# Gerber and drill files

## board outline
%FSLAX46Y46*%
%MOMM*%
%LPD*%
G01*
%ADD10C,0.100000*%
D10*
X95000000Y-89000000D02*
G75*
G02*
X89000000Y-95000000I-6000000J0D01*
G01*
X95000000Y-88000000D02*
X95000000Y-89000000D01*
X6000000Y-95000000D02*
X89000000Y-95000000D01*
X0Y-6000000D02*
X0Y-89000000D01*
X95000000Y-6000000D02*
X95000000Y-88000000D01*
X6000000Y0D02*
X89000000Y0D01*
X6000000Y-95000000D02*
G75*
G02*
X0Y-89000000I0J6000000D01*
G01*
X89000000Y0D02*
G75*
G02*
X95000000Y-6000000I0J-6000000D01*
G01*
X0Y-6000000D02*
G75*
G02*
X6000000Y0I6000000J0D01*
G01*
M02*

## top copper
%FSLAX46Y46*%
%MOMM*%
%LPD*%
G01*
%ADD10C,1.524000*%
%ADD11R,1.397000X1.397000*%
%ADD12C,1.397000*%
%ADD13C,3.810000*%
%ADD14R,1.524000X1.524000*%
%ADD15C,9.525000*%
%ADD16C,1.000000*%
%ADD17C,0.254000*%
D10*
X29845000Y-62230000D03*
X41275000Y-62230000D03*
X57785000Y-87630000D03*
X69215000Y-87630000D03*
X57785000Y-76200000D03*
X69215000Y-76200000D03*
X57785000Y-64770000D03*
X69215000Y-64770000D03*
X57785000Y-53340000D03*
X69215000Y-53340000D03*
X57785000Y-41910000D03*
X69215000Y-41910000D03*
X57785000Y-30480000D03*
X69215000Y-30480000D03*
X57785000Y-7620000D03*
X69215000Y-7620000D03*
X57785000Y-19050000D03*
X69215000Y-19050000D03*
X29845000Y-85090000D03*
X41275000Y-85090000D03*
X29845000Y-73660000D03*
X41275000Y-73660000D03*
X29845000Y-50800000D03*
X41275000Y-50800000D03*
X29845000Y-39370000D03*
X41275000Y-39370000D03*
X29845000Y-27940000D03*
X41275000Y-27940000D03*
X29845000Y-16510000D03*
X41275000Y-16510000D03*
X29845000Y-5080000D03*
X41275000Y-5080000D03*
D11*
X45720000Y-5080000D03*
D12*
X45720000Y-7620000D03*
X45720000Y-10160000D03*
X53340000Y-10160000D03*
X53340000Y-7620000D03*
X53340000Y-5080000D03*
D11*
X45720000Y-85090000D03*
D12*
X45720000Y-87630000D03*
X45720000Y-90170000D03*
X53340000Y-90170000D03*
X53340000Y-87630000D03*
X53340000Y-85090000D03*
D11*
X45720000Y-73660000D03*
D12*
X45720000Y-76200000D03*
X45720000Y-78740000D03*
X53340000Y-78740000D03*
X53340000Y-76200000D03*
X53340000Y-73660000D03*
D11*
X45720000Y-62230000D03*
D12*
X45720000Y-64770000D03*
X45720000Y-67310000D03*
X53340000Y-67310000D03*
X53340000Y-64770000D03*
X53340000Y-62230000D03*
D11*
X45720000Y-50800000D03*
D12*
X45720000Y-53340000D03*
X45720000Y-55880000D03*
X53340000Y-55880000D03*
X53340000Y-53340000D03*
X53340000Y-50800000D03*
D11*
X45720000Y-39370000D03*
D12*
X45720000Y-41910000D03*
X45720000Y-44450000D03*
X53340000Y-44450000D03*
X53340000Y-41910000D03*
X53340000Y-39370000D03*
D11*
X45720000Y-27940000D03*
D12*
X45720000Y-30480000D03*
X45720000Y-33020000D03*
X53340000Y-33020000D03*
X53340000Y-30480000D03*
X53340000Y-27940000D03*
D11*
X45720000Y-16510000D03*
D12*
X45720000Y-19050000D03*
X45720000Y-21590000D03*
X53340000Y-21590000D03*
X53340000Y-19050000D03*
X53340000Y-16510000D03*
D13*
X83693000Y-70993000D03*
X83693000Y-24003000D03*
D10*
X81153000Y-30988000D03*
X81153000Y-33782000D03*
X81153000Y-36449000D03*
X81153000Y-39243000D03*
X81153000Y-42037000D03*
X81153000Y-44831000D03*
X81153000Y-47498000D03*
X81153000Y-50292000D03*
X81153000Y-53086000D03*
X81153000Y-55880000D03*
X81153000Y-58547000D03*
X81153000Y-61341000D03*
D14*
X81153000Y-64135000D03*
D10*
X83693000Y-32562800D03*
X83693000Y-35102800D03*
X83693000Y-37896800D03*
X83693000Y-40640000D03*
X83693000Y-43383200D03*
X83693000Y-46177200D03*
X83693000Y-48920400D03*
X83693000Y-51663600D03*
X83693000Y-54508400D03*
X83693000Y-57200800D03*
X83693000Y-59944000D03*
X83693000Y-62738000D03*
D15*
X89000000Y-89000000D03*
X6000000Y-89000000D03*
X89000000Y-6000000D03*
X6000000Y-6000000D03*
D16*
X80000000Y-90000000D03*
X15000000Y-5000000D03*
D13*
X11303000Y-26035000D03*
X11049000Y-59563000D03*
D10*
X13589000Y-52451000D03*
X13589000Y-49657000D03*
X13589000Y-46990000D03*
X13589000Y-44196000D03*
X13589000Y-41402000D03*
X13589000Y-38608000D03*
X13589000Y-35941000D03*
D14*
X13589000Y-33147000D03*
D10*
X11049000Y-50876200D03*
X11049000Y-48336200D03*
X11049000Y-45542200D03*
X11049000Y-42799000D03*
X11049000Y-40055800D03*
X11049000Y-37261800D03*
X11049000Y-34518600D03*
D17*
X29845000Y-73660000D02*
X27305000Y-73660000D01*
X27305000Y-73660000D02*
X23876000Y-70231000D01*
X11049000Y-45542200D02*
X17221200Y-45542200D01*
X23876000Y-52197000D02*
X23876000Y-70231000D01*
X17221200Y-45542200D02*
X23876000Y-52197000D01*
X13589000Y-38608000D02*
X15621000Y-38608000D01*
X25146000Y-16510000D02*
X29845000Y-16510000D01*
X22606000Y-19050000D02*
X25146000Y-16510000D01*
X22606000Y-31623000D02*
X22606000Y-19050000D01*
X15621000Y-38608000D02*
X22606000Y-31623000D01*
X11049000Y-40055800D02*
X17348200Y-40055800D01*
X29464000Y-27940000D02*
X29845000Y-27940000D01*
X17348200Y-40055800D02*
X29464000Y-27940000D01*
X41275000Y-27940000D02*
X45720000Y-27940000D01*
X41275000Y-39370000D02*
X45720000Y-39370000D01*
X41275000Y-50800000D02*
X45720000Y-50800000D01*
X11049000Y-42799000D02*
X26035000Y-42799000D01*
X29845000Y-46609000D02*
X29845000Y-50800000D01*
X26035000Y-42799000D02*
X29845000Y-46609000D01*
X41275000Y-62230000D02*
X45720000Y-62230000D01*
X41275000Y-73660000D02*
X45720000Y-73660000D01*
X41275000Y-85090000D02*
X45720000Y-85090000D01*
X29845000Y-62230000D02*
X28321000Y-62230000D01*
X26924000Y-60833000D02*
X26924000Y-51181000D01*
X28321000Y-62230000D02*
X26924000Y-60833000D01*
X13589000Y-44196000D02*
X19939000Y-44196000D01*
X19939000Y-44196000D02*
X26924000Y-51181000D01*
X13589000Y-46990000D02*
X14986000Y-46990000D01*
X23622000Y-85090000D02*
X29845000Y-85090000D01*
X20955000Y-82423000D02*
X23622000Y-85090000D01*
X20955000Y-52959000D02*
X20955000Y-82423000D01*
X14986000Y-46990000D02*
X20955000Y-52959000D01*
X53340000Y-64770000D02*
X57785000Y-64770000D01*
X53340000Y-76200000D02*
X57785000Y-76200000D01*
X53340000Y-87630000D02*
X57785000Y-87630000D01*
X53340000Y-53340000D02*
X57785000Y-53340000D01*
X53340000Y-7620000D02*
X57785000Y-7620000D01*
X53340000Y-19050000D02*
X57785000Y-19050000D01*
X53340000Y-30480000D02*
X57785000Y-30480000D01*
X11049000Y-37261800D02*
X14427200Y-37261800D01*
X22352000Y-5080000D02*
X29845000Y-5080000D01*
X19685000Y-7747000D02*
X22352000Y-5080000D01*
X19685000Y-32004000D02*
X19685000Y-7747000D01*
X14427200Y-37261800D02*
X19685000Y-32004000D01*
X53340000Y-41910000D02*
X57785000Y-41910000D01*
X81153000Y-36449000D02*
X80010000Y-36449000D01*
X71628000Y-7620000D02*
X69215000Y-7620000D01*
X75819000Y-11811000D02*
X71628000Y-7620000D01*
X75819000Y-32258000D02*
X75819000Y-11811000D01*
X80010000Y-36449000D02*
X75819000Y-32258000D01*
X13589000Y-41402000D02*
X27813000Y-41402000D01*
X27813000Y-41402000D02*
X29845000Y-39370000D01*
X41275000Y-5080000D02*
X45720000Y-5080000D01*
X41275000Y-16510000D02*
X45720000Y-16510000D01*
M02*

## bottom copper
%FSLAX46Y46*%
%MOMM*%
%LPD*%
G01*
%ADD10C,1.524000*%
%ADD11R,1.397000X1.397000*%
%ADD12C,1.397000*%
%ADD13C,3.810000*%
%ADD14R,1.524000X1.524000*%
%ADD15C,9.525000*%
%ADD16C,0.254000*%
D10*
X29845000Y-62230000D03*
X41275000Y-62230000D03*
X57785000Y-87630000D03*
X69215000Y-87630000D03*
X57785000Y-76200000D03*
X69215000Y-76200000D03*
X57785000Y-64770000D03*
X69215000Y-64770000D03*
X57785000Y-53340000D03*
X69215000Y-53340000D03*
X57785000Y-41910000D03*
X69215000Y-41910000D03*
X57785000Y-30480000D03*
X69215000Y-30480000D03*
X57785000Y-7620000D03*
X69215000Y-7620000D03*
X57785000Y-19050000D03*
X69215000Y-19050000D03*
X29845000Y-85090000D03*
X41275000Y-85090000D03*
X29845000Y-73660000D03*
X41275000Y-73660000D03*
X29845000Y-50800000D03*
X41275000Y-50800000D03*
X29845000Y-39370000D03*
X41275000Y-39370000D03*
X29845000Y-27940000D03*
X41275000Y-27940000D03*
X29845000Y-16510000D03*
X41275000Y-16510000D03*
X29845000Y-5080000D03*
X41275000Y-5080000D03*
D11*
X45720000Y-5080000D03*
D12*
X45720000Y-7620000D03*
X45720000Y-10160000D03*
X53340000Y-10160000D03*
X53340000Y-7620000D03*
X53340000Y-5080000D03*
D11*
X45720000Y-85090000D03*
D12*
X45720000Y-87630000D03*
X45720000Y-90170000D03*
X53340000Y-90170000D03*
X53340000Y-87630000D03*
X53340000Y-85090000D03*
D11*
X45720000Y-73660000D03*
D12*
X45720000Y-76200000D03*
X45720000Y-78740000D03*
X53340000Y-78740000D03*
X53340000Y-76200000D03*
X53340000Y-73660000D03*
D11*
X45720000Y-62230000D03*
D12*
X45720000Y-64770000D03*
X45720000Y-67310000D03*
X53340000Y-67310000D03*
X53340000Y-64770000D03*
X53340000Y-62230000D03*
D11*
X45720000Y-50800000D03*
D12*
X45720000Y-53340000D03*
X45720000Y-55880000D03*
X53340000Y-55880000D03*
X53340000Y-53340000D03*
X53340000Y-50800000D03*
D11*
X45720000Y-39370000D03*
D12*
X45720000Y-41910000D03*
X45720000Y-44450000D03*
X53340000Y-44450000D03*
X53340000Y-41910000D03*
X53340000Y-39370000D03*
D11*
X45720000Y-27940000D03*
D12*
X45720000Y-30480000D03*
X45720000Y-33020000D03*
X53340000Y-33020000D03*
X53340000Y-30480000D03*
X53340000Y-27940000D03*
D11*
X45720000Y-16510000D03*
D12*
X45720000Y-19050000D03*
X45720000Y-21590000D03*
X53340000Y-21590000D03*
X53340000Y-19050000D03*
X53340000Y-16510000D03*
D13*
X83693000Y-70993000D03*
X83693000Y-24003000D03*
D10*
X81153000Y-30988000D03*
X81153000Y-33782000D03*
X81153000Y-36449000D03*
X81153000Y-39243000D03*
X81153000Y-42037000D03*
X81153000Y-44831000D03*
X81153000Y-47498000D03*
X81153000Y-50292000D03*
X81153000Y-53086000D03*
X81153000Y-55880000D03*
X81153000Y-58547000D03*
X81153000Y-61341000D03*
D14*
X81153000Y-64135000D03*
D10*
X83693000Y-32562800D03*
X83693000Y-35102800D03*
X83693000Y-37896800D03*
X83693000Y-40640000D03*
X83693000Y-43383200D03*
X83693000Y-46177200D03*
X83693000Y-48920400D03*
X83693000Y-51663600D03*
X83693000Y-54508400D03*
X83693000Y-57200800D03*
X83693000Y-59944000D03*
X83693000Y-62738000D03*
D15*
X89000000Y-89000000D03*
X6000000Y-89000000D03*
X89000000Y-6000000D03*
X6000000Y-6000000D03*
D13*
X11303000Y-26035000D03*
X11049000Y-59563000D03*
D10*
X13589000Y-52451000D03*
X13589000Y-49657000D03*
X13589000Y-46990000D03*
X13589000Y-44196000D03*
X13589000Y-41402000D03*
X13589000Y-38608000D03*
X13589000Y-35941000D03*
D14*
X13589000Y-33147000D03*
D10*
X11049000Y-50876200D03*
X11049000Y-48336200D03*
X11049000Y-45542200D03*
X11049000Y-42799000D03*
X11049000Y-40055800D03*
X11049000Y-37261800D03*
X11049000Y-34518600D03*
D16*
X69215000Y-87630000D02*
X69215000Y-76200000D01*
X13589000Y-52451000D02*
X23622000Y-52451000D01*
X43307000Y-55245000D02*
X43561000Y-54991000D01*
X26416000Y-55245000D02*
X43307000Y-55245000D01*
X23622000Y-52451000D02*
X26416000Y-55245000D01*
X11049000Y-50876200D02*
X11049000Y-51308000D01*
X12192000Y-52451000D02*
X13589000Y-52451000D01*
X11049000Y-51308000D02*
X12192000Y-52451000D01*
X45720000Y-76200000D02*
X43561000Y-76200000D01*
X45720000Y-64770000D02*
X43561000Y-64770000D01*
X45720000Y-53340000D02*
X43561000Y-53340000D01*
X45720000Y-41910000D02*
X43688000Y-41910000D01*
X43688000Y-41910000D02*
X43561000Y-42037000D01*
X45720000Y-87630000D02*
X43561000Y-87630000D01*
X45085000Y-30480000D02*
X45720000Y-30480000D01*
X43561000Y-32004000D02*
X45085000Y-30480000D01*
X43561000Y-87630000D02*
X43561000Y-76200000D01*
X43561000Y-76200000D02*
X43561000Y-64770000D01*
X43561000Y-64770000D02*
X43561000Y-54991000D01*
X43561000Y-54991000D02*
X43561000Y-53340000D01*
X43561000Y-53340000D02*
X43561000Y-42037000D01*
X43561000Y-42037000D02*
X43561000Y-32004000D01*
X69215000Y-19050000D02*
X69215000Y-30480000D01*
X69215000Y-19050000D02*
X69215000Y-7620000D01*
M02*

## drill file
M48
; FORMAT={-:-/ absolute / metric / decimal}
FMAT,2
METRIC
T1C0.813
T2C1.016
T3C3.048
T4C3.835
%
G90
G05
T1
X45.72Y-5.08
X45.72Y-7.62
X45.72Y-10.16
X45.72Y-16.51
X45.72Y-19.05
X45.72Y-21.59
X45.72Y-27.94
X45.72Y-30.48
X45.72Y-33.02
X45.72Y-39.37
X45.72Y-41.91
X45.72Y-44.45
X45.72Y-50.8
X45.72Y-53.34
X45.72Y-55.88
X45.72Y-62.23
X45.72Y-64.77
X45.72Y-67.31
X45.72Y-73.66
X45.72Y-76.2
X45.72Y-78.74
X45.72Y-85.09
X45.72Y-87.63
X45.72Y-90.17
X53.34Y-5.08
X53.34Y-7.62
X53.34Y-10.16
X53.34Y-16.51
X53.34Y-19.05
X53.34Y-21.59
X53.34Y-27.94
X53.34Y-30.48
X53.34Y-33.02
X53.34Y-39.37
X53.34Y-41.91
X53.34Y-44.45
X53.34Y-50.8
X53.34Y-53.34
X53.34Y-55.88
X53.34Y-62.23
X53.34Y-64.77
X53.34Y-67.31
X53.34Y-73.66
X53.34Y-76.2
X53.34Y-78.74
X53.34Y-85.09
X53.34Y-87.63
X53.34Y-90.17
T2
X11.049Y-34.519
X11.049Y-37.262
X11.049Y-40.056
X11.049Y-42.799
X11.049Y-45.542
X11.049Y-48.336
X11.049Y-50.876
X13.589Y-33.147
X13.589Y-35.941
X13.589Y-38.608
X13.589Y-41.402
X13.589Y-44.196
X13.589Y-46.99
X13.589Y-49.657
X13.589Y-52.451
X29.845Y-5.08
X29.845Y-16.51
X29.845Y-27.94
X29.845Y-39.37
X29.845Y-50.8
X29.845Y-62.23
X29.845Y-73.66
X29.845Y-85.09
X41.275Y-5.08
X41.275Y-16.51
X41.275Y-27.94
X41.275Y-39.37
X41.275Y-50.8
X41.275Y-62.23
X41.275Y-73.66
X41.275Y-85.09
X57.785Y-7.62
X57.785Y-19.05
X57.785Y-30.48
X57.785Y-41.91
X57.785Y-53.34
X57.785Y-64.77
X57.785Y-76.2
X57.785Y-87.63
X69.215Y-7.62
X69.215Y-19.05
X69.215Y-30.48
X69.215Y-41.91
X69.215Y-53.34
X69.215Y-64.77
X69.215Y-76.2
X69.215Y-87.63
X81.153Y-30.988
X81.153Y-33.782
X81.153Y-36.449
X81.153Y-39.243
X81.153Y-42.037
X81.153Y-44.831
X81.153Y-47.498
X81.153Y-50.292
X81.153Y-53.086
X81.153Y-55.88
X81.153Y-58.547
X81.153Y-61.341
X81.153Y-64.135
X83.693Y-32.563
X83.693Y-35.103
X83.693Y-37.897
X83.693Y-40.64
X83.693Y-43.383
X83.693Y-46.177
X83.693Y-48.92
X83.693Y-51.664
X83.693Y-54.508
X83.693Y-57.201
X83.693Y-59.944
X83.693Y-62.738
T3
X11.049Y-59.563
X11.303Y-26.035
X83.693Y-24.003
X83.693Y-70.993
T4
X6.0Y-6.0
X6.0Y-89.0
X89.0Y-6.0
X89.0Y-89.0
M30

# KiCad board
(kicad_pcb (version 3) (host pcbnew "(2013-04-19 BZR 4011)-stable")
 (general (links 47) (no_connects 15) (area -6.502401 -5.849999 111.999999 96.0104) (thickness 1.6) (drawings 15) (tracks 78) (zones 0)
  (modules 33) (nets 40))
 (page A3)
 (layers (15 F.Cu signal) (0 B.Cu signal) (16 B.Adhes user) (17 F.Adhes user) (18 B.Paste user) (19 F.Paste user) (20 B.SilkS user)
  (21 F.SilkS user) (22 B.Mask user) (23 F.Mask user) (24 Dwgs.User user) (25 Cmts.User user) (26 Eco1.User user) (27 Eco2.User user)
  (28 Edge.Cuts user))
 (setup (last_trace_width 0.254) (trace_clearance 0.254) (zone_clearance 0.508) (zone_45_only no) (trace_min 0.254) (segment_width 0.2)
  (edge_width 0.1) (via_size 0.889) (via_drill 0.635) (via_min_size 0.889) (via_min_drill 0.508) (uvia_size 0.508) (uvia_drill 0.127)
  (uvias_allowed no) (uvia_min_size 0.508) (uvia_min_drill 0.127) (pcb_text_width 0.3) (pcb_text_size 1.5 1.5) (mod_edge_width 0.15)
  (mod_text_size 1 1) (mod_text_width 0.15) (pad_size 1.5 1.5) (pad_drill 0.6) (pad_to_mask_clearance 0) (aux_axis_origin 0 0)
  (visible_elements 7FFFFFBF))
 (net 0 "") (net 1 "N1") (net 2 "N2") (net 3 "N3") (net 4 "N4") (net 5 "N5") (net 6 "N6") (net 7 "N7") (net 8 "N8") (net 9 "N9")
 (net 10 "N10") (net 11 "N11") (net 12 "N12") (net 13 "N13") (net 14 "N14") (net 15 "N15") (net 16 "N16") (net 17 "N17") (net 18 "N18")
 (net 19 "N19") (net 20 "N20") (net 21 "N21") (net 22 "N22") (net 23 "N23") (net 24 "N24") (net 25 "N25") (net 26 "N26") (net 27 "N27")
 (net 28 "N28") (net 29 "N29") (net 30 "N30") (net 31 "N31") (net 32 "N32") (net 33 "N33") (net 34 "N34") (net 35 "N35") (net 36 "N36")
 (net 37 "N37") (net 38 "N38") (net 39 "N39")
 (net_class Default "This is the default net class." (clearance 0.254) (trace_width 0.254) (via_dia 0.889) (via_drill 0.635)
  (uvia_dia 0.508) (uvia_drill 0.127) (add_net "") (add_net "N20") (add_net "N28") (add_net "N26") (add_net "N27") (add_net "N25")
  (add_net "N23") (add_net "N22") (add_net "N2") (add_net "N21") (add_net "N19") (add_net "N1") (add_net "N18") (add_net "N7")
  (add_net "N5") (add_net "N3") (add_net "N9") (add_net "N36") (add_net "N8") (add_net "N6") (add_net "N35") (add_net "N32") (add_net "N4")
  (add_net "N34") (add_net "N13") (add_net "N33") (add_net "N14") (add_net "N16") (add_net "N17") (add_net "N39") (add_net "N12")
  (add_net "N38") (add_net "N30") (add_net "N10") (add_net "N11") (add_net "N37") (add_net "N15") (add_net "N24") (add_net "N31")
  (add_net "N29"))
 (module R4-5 (layer F.Cu) (at 35.56 62.23)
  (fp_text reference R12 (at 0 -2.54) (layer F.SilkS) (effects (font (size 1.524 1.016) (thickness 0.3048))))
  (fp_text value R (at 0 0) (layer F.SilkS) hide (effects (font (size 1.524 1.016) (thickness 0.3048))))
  (pad 1 thru_hole circle (at -5.715 0) (size 1.524 1.524) (drill 1.016) (layers *.Cu *.Mask F.SilkS) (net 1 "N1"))
  (pad 2 thru_hole circle (at 5.715 0) (size 1.524 1.524) (drill 1.016) (layers *.Cu *.Mask F.SilkS) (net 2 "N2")))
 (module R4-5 (layer F.Cu) (at 63.5 87.63)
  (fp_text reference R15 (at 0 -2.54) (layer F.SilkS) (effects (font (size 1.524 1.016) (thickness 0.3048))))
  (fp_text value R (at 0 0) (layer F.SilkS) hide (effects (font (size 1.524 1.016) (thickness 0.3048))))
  (pad 1 thru_hole circle (at -5.715 0) (size 1.524 1.524) (drill 1.016) (layers *.Cu *.Mask F.SilkS) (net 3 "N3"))
  (pad 2 thru_hole circle (at 5.715 0) (size 1.524 1.524) (drill 1.016) (layers *.Cu *.Mask F.SilkS) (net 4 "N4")))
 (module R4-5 (layer F.Cu) (at 63.5 76.2)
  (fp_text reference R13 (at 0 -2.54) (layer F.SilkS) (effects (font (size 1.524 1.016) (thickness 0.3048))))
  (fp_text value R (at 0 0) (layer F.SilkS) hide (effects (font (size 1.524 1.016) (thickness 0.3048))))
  (pad 1 thru_hole circle (at -5.715 0) (size 1.524 1.524) (drill 1.016) (layers *.Cu *.Mask F.SilkS) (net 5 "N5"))
  (pad 2 thru_hole circle (at 5.715 0) (size 1.524 1.524) (drill 1.016) (layers *.Cu *.Mask F.SilkS) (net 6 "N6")))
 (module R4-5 (layer F.Cu) (at 63.5 64.77)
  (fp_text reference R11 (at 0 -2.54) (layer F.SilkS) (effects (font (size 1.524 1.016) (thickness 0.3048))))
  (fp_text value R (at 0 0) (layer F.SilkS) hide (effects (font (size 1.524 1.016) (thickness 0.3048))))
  (pad 1 thru_hole circle (at -5.715 0) (size 1.524 1.524) (drill 1.016) (layers *.Cu *.Mask F.SilkS) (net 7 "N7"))
  (pad 2 thru_hole circle (at 5.715 0) (size 1.524 1.524) (drill 1.016) (layers *.Cu *.Mask F.SilkS)))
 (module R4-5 (layer F.Cu) (at 63.5 53.34)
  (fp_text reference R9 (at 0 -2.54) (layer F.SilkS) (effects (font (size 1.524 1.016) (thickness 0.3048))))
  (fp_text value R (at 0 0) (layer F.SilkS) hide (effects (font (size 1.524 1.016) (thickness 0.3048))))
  (pad 1 thru_hole circle (at -5.715 0) (size 1.524 1.524) (drill 1.016) (layers *.Cu *.Mask F.SilkS) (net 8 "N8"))
  (pad 2 thru_hole circle (at 5.715 0) (size 1.524 1.524) (drill 1.016) (layers *.Cu *.Mask F.SilkS) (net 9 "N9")))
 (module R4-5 (layer F.Cu) (at 63.5 41.91)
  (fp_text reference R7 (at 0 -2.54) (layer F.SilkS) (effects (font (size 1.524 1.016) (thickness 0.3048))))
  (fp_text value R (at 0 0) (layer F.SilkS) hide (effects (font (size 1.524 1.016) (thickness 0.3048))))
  (pad 1 thru_hole circle (at -5.715 0) (size 1.524 1.524) (drill 1.016) (layers *.Cu *.Mask F.SilkS) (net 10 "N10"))
  (pad 2 thru_hole circle (at 5.715 0) (size 1.524 1.524) (drill 1.016) (layers *.Cu *.Mask F.SilkS) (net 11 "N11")))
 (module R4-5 (layer F.Cu) (at 63.5 30.48)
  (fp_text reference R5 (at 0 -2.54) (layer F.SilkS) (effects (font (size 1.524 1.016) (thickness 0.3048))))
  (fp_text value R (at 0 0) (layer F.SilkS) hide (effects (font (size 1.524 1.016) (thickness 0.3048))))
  (pad 1 thru_hole circle (at -5.715 0) (size 1.524 1.524) (drill 1.016) (layers *.Cu *.Mask F.SilkS) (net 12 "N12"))
  (pad 2 thru_hole circle (at 5.715 0) (size 1.524 1.524) (drill 1.016) (layers *.Cu *.Mask F.SilkS) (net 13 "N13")))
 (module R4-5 (layer F.Cu) (at 63.5 7.62)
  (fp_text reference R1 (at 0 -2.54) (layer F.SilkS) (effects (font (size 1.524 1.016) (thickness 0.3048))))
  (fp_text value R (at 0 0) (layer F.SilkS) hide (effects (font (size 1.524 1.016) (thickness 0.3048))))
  (pad 1 thru_hole circle (at -5.715 0) (size 1.524 1.524) (drill 1.016) (layers *.Cu *.Mask F.SilkS) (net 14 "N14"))
  (pad 2 thru_hole circle (at 5.715 0) (size 1.524 1.524) (drill 1.016) (layers *.Cu *.Mask F.SilkS) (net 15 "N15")))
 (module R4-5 (layer F.Cu) (at 63.5 19.05)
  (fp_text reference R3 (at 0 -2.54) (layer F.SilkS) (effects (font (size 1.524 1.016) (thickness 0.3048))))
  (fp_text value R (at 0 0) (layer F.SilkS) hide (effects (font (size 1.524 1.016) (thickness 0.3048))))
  (pad 1 thru_hole circle (at -5.715 0) (size 1.524 1.524) (drill 1.016) (layers *.Cu *.Mask F.SilkS) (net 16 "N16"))
  (pad 2 thru_hole circle (at 5.715 0) (size 1.524 1.524) (drill 1.016) (layers *.Cu *.Mask F.SilkS) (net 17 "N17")))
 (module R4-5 (layer F.Cu) (at 35.56 85.09)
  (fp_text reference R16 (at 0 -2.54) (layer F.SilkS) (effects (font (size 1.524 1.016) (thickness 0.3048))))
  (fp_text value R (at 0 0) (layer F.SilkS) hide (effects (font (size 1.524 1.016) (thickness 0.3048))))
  (pad 1 thru_hole circle (at -5.715 0) (size 1.524 1.524) (drill 1.016) (layers *.Cu *.Mask F.SilkS) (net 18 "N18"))
  (pad 2 thru_hole circle (at 5.715 0) (size 1.524 1.524) (drill 1.016) (layers *.Cu *.Mask F.SilkS) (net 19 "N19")))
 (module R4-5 (layer F.Cu) (at 35.56 73.66)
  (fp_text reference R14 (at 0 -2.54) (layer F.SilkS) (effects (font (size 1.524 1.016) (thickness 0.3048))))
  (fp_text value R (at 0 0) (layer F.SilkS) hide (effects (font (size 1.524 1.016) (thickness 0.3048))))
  (pad 1 thru_hole circle (at -5.715 0) (size 1.524 1.524) (drill 1.016) (layers *.Cu *.Mask F.SilkS) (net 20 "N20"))
  (pad 2 thru_hole circle (at 5.715 0) (size 1.524 1.524) (drill 1.016) (layers *.Cu *.Mask F.SilkS) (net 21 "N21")))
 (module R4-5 (layer F.Cu) (at 35.56 50.8)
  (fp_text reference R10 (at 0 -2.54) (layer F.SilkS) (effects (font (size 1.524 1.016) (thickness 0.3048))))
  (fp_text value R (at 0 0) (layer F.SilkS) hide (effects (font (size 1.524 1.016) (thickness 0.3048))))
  (pad 1 thru_hole circle (at -5.715 0) (size 1.524 1.524) (drill 1.016) (layers *.Cu *.Mask F.SilkS) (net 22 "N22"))
  (pad 2 thru_hole circle (at 5.715 0) (size 1.524 1.524) (drill 1.016) (layers *.Cu *.Mask F.SilkS) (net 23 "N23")))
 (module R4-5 (layer F.Cu) (at 35.56 39.37)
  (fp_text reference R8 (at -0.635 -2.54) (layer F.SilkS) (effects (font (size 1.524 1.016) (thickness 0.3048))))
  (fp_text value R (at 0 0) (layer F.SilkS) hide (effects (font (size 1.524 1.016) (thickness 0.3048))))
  (pad 1 thru_hole circle (at -5.715 0) (size 1.524 1.524) (drill 1.016) (layers *.Cu *.Mask F.SilkS) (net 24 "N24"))
  (pad 2 thru_hole circle (at 5.715 0) (size 1.524 1.524) (drill 1.016) (layers *.Cu *.Mask F.SilkS) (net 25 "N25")))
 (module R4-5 (layer F.Cu) (at 35.56 27.94)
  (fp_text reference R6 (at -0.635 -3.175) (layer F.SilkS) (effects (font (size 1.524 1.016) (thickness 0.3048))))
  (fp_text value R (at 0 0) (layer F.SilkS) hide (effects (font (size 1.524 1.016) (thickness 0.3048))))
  (pad 1 thru_hole circle (at -5.715 0) (size 1.524 1.524) (drill 1.016) (layers *.Cu *.Mask F.SilkS) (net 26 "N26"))
  (pad 2 thru_hole circle (at 5.715 0) (size 1.524 1.524) (drill 1.016) (layers *.Cu *.Mask F.SilkS) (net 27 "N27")))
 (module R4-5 (layer F.Cu) (at 35.56 16.51)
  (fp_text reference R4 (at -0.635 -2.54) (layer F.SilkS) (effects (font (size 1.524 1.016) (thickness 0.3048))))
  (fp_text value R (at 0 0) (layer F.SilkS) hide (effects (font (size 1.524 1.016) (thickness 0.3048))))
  (pad 1 thru_hole circle (at -5.715 0) (size 1.524 1.524) (drill 1.016) (layers *.Cu *.Mask F.SilkS) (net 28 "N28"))
  (pad 2 thru_hole circle (at 5.715 0) (size 1.524 1.524) (drill 1.016) (layers *.Cu *.Mask F.SilkS) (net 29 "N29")))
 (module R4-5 (layer F.Cu) (at 35.56 5.08)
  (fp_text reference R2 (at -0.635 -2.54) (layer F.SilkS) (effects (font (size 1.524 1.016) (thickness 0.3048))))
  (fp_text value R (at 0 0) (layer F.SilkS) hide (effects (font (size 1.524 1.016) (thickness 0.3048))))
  (pad 1 thru_hole circle (at -5.715 0) (size 1.524 1.524) (drill 1.016) (layers *.Cu *.Mask F.SilkS) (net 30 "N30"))
  (pad 2 thru_hole circle (at 5.715 0) (size 1.524 1.524) (drill 1.016) (layers *.Cu *.Mask F.SilkS) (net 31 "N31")))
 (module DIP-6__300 (layer F.Cu) (at 49.53 7.62 270)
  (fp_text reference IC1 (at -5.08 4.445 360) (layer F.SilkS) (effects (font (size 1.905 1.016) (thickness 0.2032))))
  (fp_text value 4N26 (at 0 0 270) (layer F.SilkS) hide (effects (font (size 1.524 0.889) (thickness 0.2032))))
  (pad 1 thru_hole rect (at -2.54 3.81 270) (size 1.397 1.397) (drill 0.8128) (layers *.Cu *.Mask F.SilkS) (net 31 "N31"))
  (pad 2 thru_hole circle (at 0 3.81 270) (size 1.397 1.397) (drill 0.8128) (layers *.Cu *.Mask F.SilkS) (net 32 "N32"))
  (pad 3 thru_hole circle (at 2.54 3.81 270) (size 1.397 1.397) (drill 0.8128) (layers *.Cu *.Mask F.SilkS))
  (pad 4 thru_hole circle (at 2.54 -3.81 270) (size 1.397 1.397) (drill 0.8128) (layers *.Cu *.Mask F.SilkS) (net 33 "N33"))
  (pad 5 thru_hole circle (at 0 -3.81 270) (size 1.397 1.397) (drill 0.8128) (layers *.Cu *.Mask F.SilkS) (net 14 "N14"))
  (pad 6 thru_hole circle (at -2.54 -3.81 270) (size 1.397 1.397) (drill 0.8128) (layers *.Cu *.Mask F.SilkS)))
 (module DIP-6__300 (layer F.Cu) (at 49.53 87.63 270)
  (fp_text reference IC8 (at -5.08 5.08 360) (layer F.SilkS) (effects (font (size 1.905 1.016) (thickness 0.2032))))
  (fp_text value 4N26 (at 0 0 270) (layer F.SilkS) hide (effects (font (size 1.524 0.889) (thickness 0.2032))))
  (pad 1 thru_hole rect (at -2.54 3.81 270) (size 1.397 1.397) (drill 0.8128) (layers *.Cu *.Mask F.SilkS) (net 19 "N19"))
  (pad 2 thru_hole circle (at 0 3.81 270) (size 1.397 1.397) (drill 0.8128) (layers *.Cu *.Mask F.SilkS) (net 32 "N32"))
  (pad 3 thru_hole circle (at 2.54 3.81 270) (size 1.397 1.397) (drill 0.8128) (layers *.Cu *.Mask F.SilkS))
  (pad 4 thru_hole circle (at 2.54 -3.81 270) (size 1.397 1.397) (drill 0.8128) (layers *.Cu *.Mask F.SilkS) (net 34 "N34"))
  (pad 5 thru_hole circle (at 0 -3.81 270) (size 1.397 1.397) (drill 0.8128) (layers *.Cu *.Mask F.SilkS) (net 3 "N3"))
  (pad 6 thru_hole circle (at -2.54 -3.81 270) (size 1.397 1.397) (drill 0.8128) (layers *.Cu *.Mask F.SilkS)))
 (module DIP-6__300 (layer F.Cu) (at 49.53 76.2 270)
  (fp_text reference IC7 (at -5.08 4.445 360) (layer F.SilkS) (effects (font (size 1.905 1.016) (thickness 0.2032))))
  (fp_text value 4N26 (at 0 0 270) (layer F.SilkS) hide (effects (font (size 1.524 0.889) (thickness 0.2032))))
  (pad 1 thru_hole rect (at -2.54 3.81 270) (size 1.397 1.397) (drill 0.8128) (layers *.Cu *.Mask F.SilkS) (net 21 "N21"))
  (pad 2 thru_hole circle (at 0 3.81 270) (size 1.397 1.397) (drill 0.8128) (layers *.Cu *.Mask F.SilkS) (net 32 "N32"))
  (pad 3 thru_hole circle (at 2.54 3.81 270) (size 1.397 1.397) (drill 0.8128) (layers *.Cu *.Mask F.SilkS))
  (pad 4 thru_hole circle (at 2.54 -3.81 270) (size 1.397 1.397) (drill 0.8128) (layers *.Cu *.Mask F.SilkS) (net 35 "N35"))
  (pad 5 thru_hole circle (at 0 -3.81 270) (size 1.397 1.397) (drill 0.8128) (layers *.Cu *.Mask F.SilkS) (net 5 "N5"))
  (pad 6 thru_hole circle (at -2.54 -3.81 270) (size 1.397 1.397) (drill 0.8128) (layers *.Cu *.Mask F.SilkS)))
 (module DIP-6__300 (layer F.Cu) (at 49.53 64.77 270)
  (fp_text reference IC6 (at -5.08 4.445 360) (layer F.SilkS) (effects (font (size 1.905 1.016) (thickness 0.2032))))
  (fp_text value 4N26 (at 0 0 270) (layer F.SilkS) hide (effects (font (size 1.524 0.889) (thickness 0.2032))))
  (pad 1 thru_hole rect (at -2.54 3.81 270) (size 1.397 1.397) (drill 0.8128) (layers *.Cu *.Mask F.SilkS) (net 2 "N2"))
  (pad 2 thru_hole circle (at 0 3.81 270) (size 1.397 1.397) (drill 0.8128) (layers *.Cu *.Mask F.SilkS) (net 32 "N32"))
  (pad 3 thru_hole circle (at 2.54 3.81 270) (size 1.397 1.397) (drill 0.8128) (layers *.Cu *.Mask F.SilkS))
  (pad 4 thru_hole circle (at 2.54 -3.81 270) (size 1.397 1.397) (drill 0.8128) (layers *.Cu *.Mask F.SilkS))
  (pad 5 thru_hole circle (at 0 -3.81 270) (size 1.397 1.397) (drill 0.8128) (layers *.Cu *.Mask F.SilkS) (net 7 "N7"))
  (pad 6 thru_hole circle (at -2.54 -3.81 270) (size 1.397 1.397) (drill 0.8128) (layers *.Cu *.Mask F.SilkS)))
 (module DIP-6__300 (layer F.Cu) (at 49.53 53.34 270)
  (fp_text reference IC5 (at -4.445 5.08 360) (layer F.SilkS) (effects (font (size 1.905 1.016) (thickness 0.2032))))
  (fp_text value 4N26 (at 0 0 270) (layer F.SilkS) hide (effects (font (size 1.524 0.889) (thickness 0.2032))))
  (pad 1 thru_hole rect (at -2.54 3.81 270) (size 1.397 1.397) (drill 0.8128) (layers *.Cu *.Mask F.SilkS) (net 23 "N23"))
  (pad 2 thru_hole circle (at 0 3.81 270) (size 1.397 1.397) (drill 0.8128) (layers *.Cu *.Mask F.SilkS) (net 32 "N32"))
  (pad 3 thru_hole circle (at 2.54 3.81 270) (size 1.397 1.397) (drill 0.8128) (layers *.Cu *.Mask F.SilkS))
  (pad 4 thru_hole circle (at 2.54 -3.81 270) (size 1.397 1.397) (drill 0.8128) (layers *.Cu *.Mask F.SilkS) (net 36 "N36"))
  (pad 5 thru_hole circle (at 0 -3.81 270) (size 1.397 1.397) (drill 0.8128) (layers *.Cu *.Mask F.SilkS) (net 8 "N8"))
  (pad 6 thru_hole circle (at -2.54 -3.81 270) (size 1.397 1.397) (drill 0.8128) (layers *.Cu *.Mask F.SilkS)))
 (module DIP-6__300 (layer F.Cu) (at 49.53 41.91 270)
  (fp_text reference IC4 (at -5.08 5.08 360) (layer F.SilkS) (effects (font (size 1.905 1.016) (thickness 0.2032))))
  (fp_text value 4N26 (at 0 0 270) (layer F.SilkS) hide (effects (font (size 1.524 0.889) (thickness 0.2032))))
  (pad 1 thru_hole rect (at -2.54 3.81 270) (size 1.397 1.397) (drill 0.8128) (layers *.Cu *.Mask F.SilkS) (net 25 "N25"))
  (pad 2 thru_hole circle (at 0 3.81 270) (size 1.397 1.397) (drill 0.8128) (layers *.Cu *.Mask F.SilkS) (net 32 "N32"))
  (pad 3 thru_hole circle (at 2.54 3.81 270) (size 1.397 1.397) (drill 0.8128) (layers *.Cu *.Mask F.SilkS))
  (pad 4 thru_hole circle (at 2.54 -3.81 270) (size 1.397 1.397) (drill 0.8128) (layers *.Cu *.Mask F.SilkS) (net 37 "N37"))
  (pad 5 thru_hole circle (at 0 -3.81 270) (size 1.397 1.397) (drill 0.8128) (layers *.Cu *.Mask F.SilkS) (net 10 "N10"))
  (pad 6 thru_hole circle (at -2.54 -3.81 270) (size 1.397 1.397) (drill 0.8128) (layers *.Cu *.Mask F.SilkS)))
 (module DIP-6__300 (layer F.Cu) (at 49.53 30.48 270)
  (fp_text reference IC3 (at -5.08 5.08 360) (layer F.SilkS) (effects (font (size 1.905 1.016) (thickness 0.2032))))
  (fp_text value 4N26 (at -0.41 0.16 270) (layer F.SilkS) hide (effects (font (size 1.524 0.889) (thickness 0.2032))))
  (pad 1 thru_hole rect (at -2.54 3.81 270) (size 1.397 1.397) (drill 0.8128) (layers *.Cu *.Mask F.SilkS) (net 27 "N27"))
  (pad 2 thru_hole circle (at 0 3.81 270) (size 1.397 1.397) (drill 0.8128) (layers *.Cu *.Mask F.SilkS) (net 32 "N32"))
  (pad 3 thru_hole circle (at 2.54 3.81 270) (size 1.397 1.397) (drill 0.8128) (layers *.Cu *.Mask F.SilkS))
  (pad 4 thru_hole circle (at 2.54 -3.81 270) (size 1.397 1.397) (drill 0.8128) (layers *.Cu *.Mask F.SilkS) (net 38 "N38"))
  (pad 5 thru_hole circle (at 0 -3.81 270) (size 1.397 1.397) (drill 0.8128) (layers *.Cu *.Mask F.SilkS) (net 12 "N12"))
  (pad 6 thru_hole circle (at -2.54 -3.81 270) (size 1.397 1.397) (drill 0.8128) (layers *.Cu *.Mask F.SilkS)))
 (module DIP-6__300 (layer F.Cu) (at 49.53 19.05 270)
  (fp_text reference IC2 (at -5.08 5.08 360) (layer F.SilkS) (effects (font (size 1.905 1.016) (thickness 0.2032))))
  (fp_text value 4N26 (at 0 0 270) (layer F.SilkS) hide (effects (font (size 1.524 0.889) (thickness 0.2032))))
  (pad 1 thru_hole rect (at -2.54 3.81 270) (size 1.397 1.397) (drill 0.8128) (layers *.Cu *.Mask F.SilkS) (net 29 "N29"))
  (pad 2 thru_hole circle (at 0 3.81 270) (size 1.397 1.397) (drill 0.8128) (layers *.Cu *.Mask F.SilkS) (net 32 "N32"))
  (pad 3 thru_hole circle (at 2.54 3.81 270) (size 1.397 1.397) (drill 0.8128) (layers *.Cu *.Mask F.SilkS))
  (pad 4 thru_hole circle (at 2.54 -3.81 270) (size 1.397 1.397) (drill 0.8128) (layers *.Cu *.Mask F.SilkS) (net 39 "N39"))
  (pad 5 thru_hole circle (at 0 -3.81 270) (size 1.397 1.397) (drill 0.8128) (layers *.Cu *.Mask F.SilkS) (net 16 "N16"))
  (pad 6 thru_hole circle (at -2.54 -3.81 270) (size 1.397 1.397) (drill 0.8128) (layers *.Cu *.Mask F.SilkS)))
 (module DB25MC (layer F.Cu) (at 82.423 47.498 270)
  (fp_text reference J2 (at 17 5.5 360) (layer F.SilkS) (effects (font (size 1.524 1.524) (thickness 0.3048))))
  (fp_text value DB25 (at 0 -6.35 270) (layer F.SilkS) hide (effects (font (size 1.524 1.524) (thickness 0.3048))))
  (pad "" thru_hole circle (at 23.495 -1.27 270) (size 3.81 3.81) (drill 3.048) (layers *.Cu *.Mask F.SilkS))
  (pad "" thru_hole circle (at -23.495 -1.27 270) (size 3.81 3.81) (drill 3.048) (layers *.Cu *.Mask F.SilkS))
  (pad 13 thru_hole circle (at -16.51 1.27 270) (size 1.524 1.524) (drill 1.016) (layers *.Cu *.Mask F.SilkS))
  (pad 12 thru_hole circle (at -13.716 1.27 270) (size 1.524 1.524) (drill 1.016) (layers *.Cu *.Mask F.SilkS))
  (pad 11 thru_hole circle (at -11.049 1.27 270) (size 1.524 1.524) (drill 1.016) (layers *.Cu *.Mask F.SilkS) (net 15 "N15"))
  (pad 10 thru_hole circle (at -8.255 1.27 270) (size 1.524 1.524) (drill 1.016) (layers *.Cu *.Mask F.SilkS) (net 17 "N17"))
  (pad 9 thru_hole circle (at -5.461 1.27 270) (size 1.524 1.524) (drill 1.016) (layers *.Cu *.Mask F.SilkS) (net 13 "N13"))
  (pad 8 thru_hole circle (at -2.667 1.27 270) (size 1.524 1.524) (drill 1.016) (layers *.Cu *.Mask F.SilkS) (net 11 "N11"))
  (pad 7 thru_hole circle (at 0 1.27 270) (size 1.524 1.524) (drill 1.016) (layers *.Cu *.Mask F.SilkS) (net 9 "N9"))
  (pad 6 thru_hole circle (at 2.794 1.27 270) (size 1.524 1.524) (drill 1.016) (layers *.Cu *.Mask F.SilkS))
  (pad 5 thru_hole circle (at 5.588 1.27 270) (size 1.524 1.524) (drill 1.016) (layers *.Cu *.Mask F.SilkS) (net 6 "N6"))
  (pad 4 thru_hole circle (at 8.382 1.27 270) (size 1.524 1.524) (drill 1.016) (layers *.Cu *.Mask F.SilkS) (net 4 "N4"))
  (pad 3 thru_hole circle (at 11.049 1.27 270) (size 1.524 1.524) (drill 1.016) (layers *.Cu *.Mask F.SilkS))
  (pad 2 thru_hole circle (at 13.843 1.27 270) (size 1.524 1.524) (drill 1.016) (layers *.Cu *.Mask F.SilkS))
  (pad 1 thru_hole rect (at 16.637 1.27 270) (size 1.524 1.524) (drill 1.016) (layers *.Cu *.Mask F.SilkS))
  (pad 25 thru_hole circle (at -14.9352 -1.27 270) (size 1.524 1.524) (drill 1.016) (layers *.Cu *.Mask F.SilkS))
  (pad 24 thru_hole circle (at -12.3952 -1.27 270) (size 1.524 1.524) (drill 1.016) (layers *.Cu *.Mask F.SilkS))
  (pad 23 thru_hole circle (at -9.6012 -1.27 270) (size 1.524 1.524) (drill 1.016) (layers *.Cu *.Mask F.SilkS) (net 33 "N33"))
  (pad 22 thru_hole circle (at -6.858 -1.27 270) (size 1.524 1.524) (drill 1.016) (layers *.Cu *.Mask F.SilkS) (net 39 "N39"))
  (pad 21 thru_hole circle (at -4.1148 -1.27 270) (size 1.524 1.524) (drill 1.016) (layers *.Cu *.Mask F.SilkS) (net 38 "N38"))
  (pad 20 thru_hole circle (at -1.3208 -1.27 270) (size 1.524 1.524) (drill 1.016) (layers *.Cu *.Mask F.SilkS) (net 37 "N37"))
  (pad 19 thru_hole circle (at 1.4224 -1.27 270) (size 1.524 1.524) (drill 1.016) (layers *.Cu *.Mask F.SilkS) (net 36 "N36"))
  (pad 18 thru_hole circle (at 4.1656 -1.27 270) (size 1.524 1.524) (drill 1.016) (layers *.Cu *.Mask F.SilkS))
  (pad 17 thru_hole circle (at 7.0104 -1.27 270) (size 1.524 1.524) (drill 1.016) (layers *.Cu *.Mask F.SilkS) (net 35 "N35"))
  (pad 16 thru_hole circle (at 9.7028 -1.27 270) (size 1.524 1.524) (drill 1.016) (layers *.Cu *.Mask F.SilkS) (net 34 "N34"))
  (pad 15 thru_hole circle (at 12.446 -1.27 270) (size 1.524 1.524) (drill 1.016) (layers *.Cu *.Mask F.SilkS))
  (pad 14 thru_hole circle (at 15.24 -1.27 270) (size 1.524 1.524) (drill 1.016) (layers *.Cu *.Mask F.SilkS)))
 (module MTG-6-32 (layer F.Cu) (at 89 89)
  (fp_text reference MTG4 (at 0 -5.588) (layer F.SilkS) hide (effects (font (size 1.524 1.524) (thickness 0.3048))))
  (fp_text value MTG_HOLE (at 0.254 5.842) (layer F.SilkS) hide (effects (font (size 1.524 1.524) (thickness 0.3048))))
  (pad 1 thru_hole circle (at 0 0) (size 9.525 9.525) (drill 3.8354) (layers *.Cu *.Mask)))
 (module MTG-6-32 (layer F.Cu) (at 6 89)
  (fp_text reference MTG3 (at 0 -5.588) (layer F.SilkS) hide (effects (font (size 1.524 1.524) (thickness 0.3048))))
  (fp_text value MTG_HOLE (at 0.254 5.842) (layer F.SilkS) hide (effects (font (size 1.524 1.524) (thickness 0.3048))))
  (pad 1 thru_hole circle (at 0 0) (size 9.525 9.525) (drill 3.8354) (layers *.Cu *.Mask)))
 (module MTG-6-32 (layer F.Cu) (at 89 6)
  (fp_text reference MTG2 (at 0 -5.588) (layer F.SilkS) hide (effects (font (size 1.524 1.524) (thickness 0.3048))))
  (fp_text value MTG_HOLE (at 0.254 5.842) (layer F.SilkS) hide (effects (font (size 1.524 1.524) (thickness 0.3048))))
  (pad 1 thru_hole circle (at 0 0) (size 9.525 9.525) (drill 3.8354) (layers *.Cu *.Mask)))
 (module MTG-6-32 (layer F.Cu) (at 6 6)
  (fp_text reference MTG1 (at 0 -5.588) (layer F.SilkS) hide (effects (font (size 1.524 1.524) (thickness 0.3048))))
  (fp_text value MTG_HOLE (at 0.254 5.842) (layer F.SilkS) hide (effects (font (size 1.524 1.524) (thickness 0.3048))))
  (pad 1 thru_hole circle (at 0 0) (size 9.525 9.525) (drill 3.8354) (layers *.Cu *.Mask)))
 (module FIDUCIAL (layer F.Cu) (at 80 90)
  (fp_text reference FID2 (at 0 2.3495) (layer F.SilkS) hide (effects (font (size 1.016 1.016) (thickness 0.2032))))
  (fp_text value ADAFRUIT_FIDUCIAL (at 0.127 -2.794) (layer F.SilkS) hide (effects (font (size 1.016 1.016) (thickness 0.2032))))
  (pad 1 smd circle (at 0 0) (size 1 1) (layers F.Cu F.Paste F.Mask) (solder_mask_margin 1) (clearance 1)))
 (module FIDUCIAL (layer F.Cu) (at 15 5)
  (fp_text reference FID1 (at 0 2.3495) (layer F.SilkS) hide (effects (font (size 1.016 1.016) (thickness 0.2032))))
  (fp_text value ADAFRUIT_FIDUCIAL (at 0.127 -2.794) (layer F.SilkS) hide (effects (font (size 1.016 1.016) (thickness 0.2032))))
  (pad 1 smd circle (at 0 0) (size 1 1) (layers F.Cu F.Paste F.Mask) (solder_mask_margin 1) (clearance 1)))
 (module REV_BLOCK (layer F.Cu) (at 77.851 82.296)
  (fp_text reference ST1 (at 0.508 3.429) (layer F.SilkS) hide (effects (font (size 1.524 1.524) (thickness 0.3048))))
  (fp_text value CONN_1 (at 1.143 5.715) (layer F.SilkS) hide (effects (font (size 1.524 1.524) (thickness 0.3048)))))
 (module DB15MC (layer F.Cu) (at 12.319 42.799 90)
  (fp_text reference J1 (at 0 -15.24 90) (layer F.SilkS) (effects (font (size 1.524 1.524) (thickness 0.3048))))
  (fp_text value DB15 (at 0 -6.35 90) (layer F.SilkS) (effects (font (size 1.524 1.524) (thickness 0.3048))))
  (pad "" thru_hole circle (at 16.764 -1.016 90) (size 3.81 3.81) (drill 3.048) (layers *.Cu *.Mask F.SilkS))
  (pad "" thru_hole circle (at -16.764 -1.27 90) (size 3.81 3.81) (drill 3.048) (layers *.Cu *.Mask F.SilkS))
  (pad 8 thru_hole circle (at -9.652 1.27 90) (size 1.524 1.524) (drill 1.016) (layers *.Cu *.Mask F.SilkS) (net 32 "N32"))
  (pad 7 thru_hole circle (at -6.858 1.27 90) (size 1.524 1.524) (drill 1.016) (layers *.Cu *.Mask F.SilkS))
  (pad 6 thru_hole circle (at -4.191 1.27 90) (size 1.524 1.524) (drill 1.016) (layers *.Cu *.Mask F.SilkS) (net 18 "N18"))
  (pad 5 thru_hole circle (at -1.397 1.27 90) (size 1.524 1.524) (drill 1.016) (layers *.Cu *.Mask F.SilkS) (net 1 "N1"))
  (pad 4 thru_hole circle (at 1.397 1.27 90) (size 1.524 1.524) (drill 1.016) (layers *.Cu *.Mask F.SilkS) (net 24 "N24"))
  (pad 3 thru_hole circle (at 4.191 1.27 90) (size 1.524 1.524) (drill 1.016) (layers *.Cu *.Mask F.SilkS) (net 28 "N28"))
  (pad 2 thru_hole circle (at 6.858 1.27 90) (size 1.524 1.524) (drill 1.016) (layers *.Cu *.Mask F.SilkS))
  (pad 1 thru_hole rect (at 9.652 1.27 90) (size 1.524 1.524) (drill 1.016) (layers *.Cu *.Mask F.SilkS))
  (pad 15 thru_hole circle (at -8.0772 -1.27 90) (size 1.524 1.524) (drill 1.016) (layers *.Cu *.Mask F.SilkS) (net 32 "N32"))
  (pad 14 thru_hole circle (at -5.5372 -1.27 90) (size 1.524 1.524) (drill 1.016) (layers *.Cu *.Mask F.SilkS))
  (pad 13 thru_hole circle (at -2.7432 -1.27 90) (size 1.524 1.524) (drill 1.016) (layers *.Cu *.Mask F.SilkS) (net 20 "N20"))
  (pad 12 thru_hole circle (at 0 -1.27 90) (size 1.524 1.524) (drill 1.016) (layers *.Cu *.Mask F.SilkS) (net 22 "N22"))
  (pad 11 thru_hole circle (at 2.7432 -1.27 90) (size 1.524 1.524) (drill 1.016) (layers *.Cu *.Mask F.SilkS) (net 26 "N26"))
  (pad 10 thru_hole circle (at 5.5372 -1.27 90) (size 1.524 1.524) (drill 1.016) (layers *.Cu *.Mask F.SilkS) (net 30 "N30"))
  (pad 9 thru_hole circle (at 8.2804 -1.27 90) (size 1.524 1.524) (drill 1.016) (layers *.Cu *.Mask F.SilkS)))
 (gr_arc (start 89 89) (end 95 89) (angle 90) (layer Edge.Cuts) (width 0.1))
 (gr_line (start 95 88) (end 95 89) (angle 90) (layer Edge.Cuts) (width 0.1))
 (gr_line (start 6 95) (end 89 95) (angle 90) (layer Edge.Cuts) (width 0.1))
 (gr_line (start 0 6) (end 0 89) (angle 90) (layer Edge.Cuts) (width 0.1))
 (gr_line (start 95 6) (end 95 88) (angle 90) (layer Edge.Cuts) (width 0.1))
 (gr_line (start 6 0) (end 89 0) (angle 90) (layer Edge.Cuts) (width 0.1))
 (gr_arc (start 6 89) (end 6 95) (angle 90) (layer Edge.Cuts) (width 0.1))
 (gr_arc (start 89 6) (end 89 0) (angle 90) (layer Edge.Cuts) (width 0.1))
 (gr_arc (start 6 6) (end 0 6) (angle 90) (layer Edge.Cuts) (width 0.1))
 (segment (start 29.845 73.66) (end 27.305 73.66) (width 0.254) (layer F.Cu) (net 20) (status 400010))
 (segment (start 27.305 73.66) (end 23.876 70.231) (width 0.254) (layer F.Cu) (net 20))
 (segment (start 11.049 45.5422) (end 17.2212 45.5422) (width 0.254) (layer F.Cu) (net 20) (status 400010))
 (segment (start 23.876 52.197) (end 23.876 70.231) (width 0.254) (layer F.Cu) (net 20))
 (segment (start 17.2212 45.5422) (end 23.876 52.197) (width 0.254) (layer F.Cu) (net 20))
 (segment (start 13.589 38.608) (end 15.621 38.608) (width 0.254) (layer F.Cu) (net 28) (status 400010))
 (segment (start 25.146 16.51) (end 29.845 16.51) (width 0.254) (layer F.Cu) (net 28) (status 800020))
 (segment (start 22.606 19.05) (end 25.146 16.51) (width 0.254) (layer F.Cu) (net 28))
 (segment (start 22.606 31.623) (end 22.606 19.05) (width 0.254) (layer F.Cu) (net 28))
 (segment (start 15.621 38.608) (end 22.606 31.623) (width 0.254) (layer F.Cu) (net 28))
 (segment (start 11.049 40.0558) (end 17.3482 40.0558) (width 0.254) (layer F.Cu) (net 26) (status 400010))
 (segment (start 29.464 27.94) (end 29.845 27.94) (width 0.254) (layer F.Cu) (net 26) (status C00030))
 (segment (start 17.3482 40.0558) (end 29.464 27.94) (width 0.254) (layer F.Cu) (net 26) (status 800020))
 (segment (start 41.275 27.94) (end 45.72 27.94) (width 0.254) (layer F.Cu) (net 27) (status 30))
 (segment (start 41.275 39.37) (end 45.72 39.37) (width 0.254) (layer F.Cu) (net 25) (status 30))
 (segment (start 41.275 50.8) (end 45.72 50.8) (width 0.254) (layer F.Cu) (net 23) (status 30))
 (segment (start 11.049 42.799) (end 26.035 42.799) (width 0.254) (layer F.Cu) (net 22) (status 400010))
 (segment (start 29.845 46.609) (end 29.845 50.8) (width 0.254) (layer F.Cu) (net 22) (status 800020))
 (segment (start 26.035 42.799) (end 29.845 46.609) (width 0.254) (layer F.Cu) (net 22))
 (segment (start 41.275 62.23) (end 45.72 62.23) (width 0.254) (layer F.Cu) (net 2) (status 30))
 (segment (start 41.275 73.66) (end 45.72 73.66) (width 0.254) (layer F.Cu) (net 21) (status 30))
 (segment (start 41.275 85.09) (end 45.72 85.09) (width 0.254) (layer F.Cu) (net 19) (status 30))
 (segment (start 29.845 62.23) (end 28.321 62.23) (width 0.254) (layer F.Cu) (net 1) (status 400010))
 (segment (start 26.924 60.833) (end 26.924 51.181) (width 0.254) (layer F.Cu) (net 1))
 (segment (start 28.321 62.23) (end 26.924 60.833) (width 0.254) (layer F.Cu) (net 1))
 (segment (start 13.589 44.196) (end 19.939 44.196) (width 0.254) (layer F.Cu) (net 1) (status 400010))
 (segment (start 19.939 44.196) (end 26.924 51.181) (width 0.254) (layer F.Cu) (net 1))
 (segment (start 13.589 46.99) (end 14.986 46.99) (width 0.254) (layer F.Cu) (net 18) (status 400010))
 (segment (start 23.622 85.09) (end 29.845 85.09) (width 0.254) (layer F.Cu) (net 18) (status 800020))
 (segment (start 20.955 82.423) (end 23.622 85.09) (width 0.254) (layer F.Cu) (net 18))
 (segment (start 20.955 52.959) (end 20.955 82.423) (width 0.254) (layer F.Cu) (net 18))
 (segment (start 14.986 46.99) (end 20.955 52.959) (width 0.254) (layer F.Cu) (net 18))
 (segment (start 53.34 64.77) (end 57.785 64.77) (width 0.254) (layer F.Cu) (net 7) (status 30))
 (segment (start 53.34 76.2) (end 57.785 76.2) (width 0.254) (layer F.Cu) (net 5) (status 30))
 (segment (start 53.34 87.63) (end 57.785 87.63) (width 0.254) (layer F.Cu) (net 3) (status 30))
 (segment (start 53.34 53.34) (end 57.785 53.34) (width 0.254) (layer F.Cu) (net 8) (status 30))
 (segment (start 69.215 87.63) (end 69.215 76.2) (width 0.254) (layer B.Cu) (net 6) (status 30))
 (segment (start 13.589 52.451) (end 23.622 52.451) (width 0.254) (layer B.Cu) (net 32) (status 400010))
 (segment (start 43.307 55.245) (end 43.561 54.991) (width 0.254) (layer B.Cu) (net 32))
 (segment (start 26.416 55.245) (end 43.307 55.245) (width 0.254) (layer B.Cu) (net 32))
 (segment (start 23.622 52.451) (end 26.416 55.245) (width 0.254) (layer B.Cu) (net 32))
 (segment (start 11.049 50.8762) (end 11.049 51.308) (width 0.254) (layer B.Cu) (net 32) (status C00030))
 (segment (start 12.192 52.451) (end 13.589 52.451) (width 0.254) (layer B.Cu) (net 32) (status 800020))
 (segment (start 11.049 51.308) (end 12.192 52.451) (width 0.254) (layer B.Cu) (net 32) (status 400010))
 (segment (start 45.72 76.2) (end 43.561 76.2) (width 0.254) (layer B.Cu) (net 32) (status 400010))
 (segment (start 45.72 64.77) (end 43.561 64.77) (width 0.254) (layer B.Cu) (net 32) (status 400010))
 (segment (start 45.72 53.34) (end 43.561 53.34) (width 0.254) (layer B.Cu) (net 32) (status 400010))
 (segment (start 45.72 41.91) (end 43.688 41.91) (width 0.254) (layer B.Cu) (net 32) (status 400010))
 (segment (start 43.688 41.91) (end 43.561 42.037) (width 0.254) (layer B.Cu) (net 32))
 (segment (start 45.72 87.63) (end 43.561 87.63) (width 0.254) (layer B.Cu) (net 32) (status 400010))
 (segment (start 45.085 30.48) (end 45.72 30.48) (width 0.254) (layer B.Cu) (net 32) (status C00030))
 (segment (start 43.561 32.004) (end 45.085 30.48) (width 0.254) (layer B.Cu) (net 32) (status 800020))
 (segment (start 43.561 87.63) (end 43.561 76.2) (width 0.254) (layer B.Cu) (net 32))
 (segment (start 43.561 76.2) (end 43.561 64.77) (width 0.254) (layer B.Cu) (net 32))
 (segment (start 43.561 64.77) (end 43.561 54.991) (width 0.254) (layer B.Cu) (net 32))
 (segment (start 43.561 54.991) (end 43.561 53.34) (width 0.254) (layer B.Cu) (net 32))
 (segment (start 43.561 53.34) (end 43.561 42.037) (width 0.254) (layer B.Cu) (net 32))
 (segment (start 43.561 42.037) (end 43.561 32.004) (width 0.254) (layer B.Cu) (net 32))
 (segment (start 53.34 7.62) (end 57.785 7.62) (width 0.254) (layer F.Cu) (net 14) (status 30))
 (segment (start 53.34 19.05) (end 57.785 19.05) (width 0.254) (layer F.Cu) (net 16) (status 30))
 (segment (start 69.215 19.05) (end 69.215 30.48) (width 0.254) (layer B.Cu) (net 17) (status 30))
 (segment (start 53.34 30.48) (end 57.785 30.48) (width 0.254) (layer F.Cu) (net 12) (status 30))
 (segment (start 11.049 37.2618) (end 14.4272 37.2618) (width 0.254) (layer F.Cu) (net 30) (status 400010))
 (segment (start 22.352 5.08) (end 29.845 5.08) (width 0.254) (layer F.Cu) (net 30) (status 800020))
 (segment (start 19.685 7.747) (end 22.352 5.08) (width 0.254) (layer F.Cu) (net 30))
 (segment (start 19.685 32.004) (end 19.685 7.747) (width 0.254) (layer F.Cu) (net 30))
 (segment (start 14.4272 37.2618) (end 19.685 32.004) (width 0.254) (layer F.Cu) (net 30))
 (segment (start 53.34 41.91) (end 57.785 41.91) (width 0.254) (layer F.Cu) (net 10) (status 30))
 (segment (start 81.153 36.449) (end 80.01 36.449) (width 0.254) (layer F.Cu) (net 15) (status 400010))
 (segment (start 71.628 7.62) (end 69.215 7.62) (width 0.254) (layer F.Cu) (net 15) (status 800020))
 (segment (start 75.819 11.811) (end 71.628 7.62) (width 0.254) (layer F.Cu) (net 15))
 (segment (start 75.819 32.258) (end 75.819 11.811) (width 0.254) (layer F.Cu) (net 15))
 (segment (start 80.01 36.449) (end 75.819 32.258) (width 0.254) (layer F.Cu) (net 15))
 (segment (start 69.215 19.05) (end 69.215 7.62) (width 0.254) (layer B.Cu) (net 15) (status 30))
 (segment (start 13.589 41.402) (end 27.813 41.402) (width 0.254) (layer F.Cu) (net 24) (status 400010))
 (segment (start 27.813 41.402) (end 29.845 39.37) (width 0.254) (layer F.Cu) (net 24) (status 800020))
 (segment (start 41.275 5.08) (end 45.72 5.08) (width 0.254) (layer F.Cu) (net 31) (status 30))
 (segment (start 41.275 16.51) (end 45.72 16.51) (width 0.254) (layer F.Cu) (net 29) (status 30)))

